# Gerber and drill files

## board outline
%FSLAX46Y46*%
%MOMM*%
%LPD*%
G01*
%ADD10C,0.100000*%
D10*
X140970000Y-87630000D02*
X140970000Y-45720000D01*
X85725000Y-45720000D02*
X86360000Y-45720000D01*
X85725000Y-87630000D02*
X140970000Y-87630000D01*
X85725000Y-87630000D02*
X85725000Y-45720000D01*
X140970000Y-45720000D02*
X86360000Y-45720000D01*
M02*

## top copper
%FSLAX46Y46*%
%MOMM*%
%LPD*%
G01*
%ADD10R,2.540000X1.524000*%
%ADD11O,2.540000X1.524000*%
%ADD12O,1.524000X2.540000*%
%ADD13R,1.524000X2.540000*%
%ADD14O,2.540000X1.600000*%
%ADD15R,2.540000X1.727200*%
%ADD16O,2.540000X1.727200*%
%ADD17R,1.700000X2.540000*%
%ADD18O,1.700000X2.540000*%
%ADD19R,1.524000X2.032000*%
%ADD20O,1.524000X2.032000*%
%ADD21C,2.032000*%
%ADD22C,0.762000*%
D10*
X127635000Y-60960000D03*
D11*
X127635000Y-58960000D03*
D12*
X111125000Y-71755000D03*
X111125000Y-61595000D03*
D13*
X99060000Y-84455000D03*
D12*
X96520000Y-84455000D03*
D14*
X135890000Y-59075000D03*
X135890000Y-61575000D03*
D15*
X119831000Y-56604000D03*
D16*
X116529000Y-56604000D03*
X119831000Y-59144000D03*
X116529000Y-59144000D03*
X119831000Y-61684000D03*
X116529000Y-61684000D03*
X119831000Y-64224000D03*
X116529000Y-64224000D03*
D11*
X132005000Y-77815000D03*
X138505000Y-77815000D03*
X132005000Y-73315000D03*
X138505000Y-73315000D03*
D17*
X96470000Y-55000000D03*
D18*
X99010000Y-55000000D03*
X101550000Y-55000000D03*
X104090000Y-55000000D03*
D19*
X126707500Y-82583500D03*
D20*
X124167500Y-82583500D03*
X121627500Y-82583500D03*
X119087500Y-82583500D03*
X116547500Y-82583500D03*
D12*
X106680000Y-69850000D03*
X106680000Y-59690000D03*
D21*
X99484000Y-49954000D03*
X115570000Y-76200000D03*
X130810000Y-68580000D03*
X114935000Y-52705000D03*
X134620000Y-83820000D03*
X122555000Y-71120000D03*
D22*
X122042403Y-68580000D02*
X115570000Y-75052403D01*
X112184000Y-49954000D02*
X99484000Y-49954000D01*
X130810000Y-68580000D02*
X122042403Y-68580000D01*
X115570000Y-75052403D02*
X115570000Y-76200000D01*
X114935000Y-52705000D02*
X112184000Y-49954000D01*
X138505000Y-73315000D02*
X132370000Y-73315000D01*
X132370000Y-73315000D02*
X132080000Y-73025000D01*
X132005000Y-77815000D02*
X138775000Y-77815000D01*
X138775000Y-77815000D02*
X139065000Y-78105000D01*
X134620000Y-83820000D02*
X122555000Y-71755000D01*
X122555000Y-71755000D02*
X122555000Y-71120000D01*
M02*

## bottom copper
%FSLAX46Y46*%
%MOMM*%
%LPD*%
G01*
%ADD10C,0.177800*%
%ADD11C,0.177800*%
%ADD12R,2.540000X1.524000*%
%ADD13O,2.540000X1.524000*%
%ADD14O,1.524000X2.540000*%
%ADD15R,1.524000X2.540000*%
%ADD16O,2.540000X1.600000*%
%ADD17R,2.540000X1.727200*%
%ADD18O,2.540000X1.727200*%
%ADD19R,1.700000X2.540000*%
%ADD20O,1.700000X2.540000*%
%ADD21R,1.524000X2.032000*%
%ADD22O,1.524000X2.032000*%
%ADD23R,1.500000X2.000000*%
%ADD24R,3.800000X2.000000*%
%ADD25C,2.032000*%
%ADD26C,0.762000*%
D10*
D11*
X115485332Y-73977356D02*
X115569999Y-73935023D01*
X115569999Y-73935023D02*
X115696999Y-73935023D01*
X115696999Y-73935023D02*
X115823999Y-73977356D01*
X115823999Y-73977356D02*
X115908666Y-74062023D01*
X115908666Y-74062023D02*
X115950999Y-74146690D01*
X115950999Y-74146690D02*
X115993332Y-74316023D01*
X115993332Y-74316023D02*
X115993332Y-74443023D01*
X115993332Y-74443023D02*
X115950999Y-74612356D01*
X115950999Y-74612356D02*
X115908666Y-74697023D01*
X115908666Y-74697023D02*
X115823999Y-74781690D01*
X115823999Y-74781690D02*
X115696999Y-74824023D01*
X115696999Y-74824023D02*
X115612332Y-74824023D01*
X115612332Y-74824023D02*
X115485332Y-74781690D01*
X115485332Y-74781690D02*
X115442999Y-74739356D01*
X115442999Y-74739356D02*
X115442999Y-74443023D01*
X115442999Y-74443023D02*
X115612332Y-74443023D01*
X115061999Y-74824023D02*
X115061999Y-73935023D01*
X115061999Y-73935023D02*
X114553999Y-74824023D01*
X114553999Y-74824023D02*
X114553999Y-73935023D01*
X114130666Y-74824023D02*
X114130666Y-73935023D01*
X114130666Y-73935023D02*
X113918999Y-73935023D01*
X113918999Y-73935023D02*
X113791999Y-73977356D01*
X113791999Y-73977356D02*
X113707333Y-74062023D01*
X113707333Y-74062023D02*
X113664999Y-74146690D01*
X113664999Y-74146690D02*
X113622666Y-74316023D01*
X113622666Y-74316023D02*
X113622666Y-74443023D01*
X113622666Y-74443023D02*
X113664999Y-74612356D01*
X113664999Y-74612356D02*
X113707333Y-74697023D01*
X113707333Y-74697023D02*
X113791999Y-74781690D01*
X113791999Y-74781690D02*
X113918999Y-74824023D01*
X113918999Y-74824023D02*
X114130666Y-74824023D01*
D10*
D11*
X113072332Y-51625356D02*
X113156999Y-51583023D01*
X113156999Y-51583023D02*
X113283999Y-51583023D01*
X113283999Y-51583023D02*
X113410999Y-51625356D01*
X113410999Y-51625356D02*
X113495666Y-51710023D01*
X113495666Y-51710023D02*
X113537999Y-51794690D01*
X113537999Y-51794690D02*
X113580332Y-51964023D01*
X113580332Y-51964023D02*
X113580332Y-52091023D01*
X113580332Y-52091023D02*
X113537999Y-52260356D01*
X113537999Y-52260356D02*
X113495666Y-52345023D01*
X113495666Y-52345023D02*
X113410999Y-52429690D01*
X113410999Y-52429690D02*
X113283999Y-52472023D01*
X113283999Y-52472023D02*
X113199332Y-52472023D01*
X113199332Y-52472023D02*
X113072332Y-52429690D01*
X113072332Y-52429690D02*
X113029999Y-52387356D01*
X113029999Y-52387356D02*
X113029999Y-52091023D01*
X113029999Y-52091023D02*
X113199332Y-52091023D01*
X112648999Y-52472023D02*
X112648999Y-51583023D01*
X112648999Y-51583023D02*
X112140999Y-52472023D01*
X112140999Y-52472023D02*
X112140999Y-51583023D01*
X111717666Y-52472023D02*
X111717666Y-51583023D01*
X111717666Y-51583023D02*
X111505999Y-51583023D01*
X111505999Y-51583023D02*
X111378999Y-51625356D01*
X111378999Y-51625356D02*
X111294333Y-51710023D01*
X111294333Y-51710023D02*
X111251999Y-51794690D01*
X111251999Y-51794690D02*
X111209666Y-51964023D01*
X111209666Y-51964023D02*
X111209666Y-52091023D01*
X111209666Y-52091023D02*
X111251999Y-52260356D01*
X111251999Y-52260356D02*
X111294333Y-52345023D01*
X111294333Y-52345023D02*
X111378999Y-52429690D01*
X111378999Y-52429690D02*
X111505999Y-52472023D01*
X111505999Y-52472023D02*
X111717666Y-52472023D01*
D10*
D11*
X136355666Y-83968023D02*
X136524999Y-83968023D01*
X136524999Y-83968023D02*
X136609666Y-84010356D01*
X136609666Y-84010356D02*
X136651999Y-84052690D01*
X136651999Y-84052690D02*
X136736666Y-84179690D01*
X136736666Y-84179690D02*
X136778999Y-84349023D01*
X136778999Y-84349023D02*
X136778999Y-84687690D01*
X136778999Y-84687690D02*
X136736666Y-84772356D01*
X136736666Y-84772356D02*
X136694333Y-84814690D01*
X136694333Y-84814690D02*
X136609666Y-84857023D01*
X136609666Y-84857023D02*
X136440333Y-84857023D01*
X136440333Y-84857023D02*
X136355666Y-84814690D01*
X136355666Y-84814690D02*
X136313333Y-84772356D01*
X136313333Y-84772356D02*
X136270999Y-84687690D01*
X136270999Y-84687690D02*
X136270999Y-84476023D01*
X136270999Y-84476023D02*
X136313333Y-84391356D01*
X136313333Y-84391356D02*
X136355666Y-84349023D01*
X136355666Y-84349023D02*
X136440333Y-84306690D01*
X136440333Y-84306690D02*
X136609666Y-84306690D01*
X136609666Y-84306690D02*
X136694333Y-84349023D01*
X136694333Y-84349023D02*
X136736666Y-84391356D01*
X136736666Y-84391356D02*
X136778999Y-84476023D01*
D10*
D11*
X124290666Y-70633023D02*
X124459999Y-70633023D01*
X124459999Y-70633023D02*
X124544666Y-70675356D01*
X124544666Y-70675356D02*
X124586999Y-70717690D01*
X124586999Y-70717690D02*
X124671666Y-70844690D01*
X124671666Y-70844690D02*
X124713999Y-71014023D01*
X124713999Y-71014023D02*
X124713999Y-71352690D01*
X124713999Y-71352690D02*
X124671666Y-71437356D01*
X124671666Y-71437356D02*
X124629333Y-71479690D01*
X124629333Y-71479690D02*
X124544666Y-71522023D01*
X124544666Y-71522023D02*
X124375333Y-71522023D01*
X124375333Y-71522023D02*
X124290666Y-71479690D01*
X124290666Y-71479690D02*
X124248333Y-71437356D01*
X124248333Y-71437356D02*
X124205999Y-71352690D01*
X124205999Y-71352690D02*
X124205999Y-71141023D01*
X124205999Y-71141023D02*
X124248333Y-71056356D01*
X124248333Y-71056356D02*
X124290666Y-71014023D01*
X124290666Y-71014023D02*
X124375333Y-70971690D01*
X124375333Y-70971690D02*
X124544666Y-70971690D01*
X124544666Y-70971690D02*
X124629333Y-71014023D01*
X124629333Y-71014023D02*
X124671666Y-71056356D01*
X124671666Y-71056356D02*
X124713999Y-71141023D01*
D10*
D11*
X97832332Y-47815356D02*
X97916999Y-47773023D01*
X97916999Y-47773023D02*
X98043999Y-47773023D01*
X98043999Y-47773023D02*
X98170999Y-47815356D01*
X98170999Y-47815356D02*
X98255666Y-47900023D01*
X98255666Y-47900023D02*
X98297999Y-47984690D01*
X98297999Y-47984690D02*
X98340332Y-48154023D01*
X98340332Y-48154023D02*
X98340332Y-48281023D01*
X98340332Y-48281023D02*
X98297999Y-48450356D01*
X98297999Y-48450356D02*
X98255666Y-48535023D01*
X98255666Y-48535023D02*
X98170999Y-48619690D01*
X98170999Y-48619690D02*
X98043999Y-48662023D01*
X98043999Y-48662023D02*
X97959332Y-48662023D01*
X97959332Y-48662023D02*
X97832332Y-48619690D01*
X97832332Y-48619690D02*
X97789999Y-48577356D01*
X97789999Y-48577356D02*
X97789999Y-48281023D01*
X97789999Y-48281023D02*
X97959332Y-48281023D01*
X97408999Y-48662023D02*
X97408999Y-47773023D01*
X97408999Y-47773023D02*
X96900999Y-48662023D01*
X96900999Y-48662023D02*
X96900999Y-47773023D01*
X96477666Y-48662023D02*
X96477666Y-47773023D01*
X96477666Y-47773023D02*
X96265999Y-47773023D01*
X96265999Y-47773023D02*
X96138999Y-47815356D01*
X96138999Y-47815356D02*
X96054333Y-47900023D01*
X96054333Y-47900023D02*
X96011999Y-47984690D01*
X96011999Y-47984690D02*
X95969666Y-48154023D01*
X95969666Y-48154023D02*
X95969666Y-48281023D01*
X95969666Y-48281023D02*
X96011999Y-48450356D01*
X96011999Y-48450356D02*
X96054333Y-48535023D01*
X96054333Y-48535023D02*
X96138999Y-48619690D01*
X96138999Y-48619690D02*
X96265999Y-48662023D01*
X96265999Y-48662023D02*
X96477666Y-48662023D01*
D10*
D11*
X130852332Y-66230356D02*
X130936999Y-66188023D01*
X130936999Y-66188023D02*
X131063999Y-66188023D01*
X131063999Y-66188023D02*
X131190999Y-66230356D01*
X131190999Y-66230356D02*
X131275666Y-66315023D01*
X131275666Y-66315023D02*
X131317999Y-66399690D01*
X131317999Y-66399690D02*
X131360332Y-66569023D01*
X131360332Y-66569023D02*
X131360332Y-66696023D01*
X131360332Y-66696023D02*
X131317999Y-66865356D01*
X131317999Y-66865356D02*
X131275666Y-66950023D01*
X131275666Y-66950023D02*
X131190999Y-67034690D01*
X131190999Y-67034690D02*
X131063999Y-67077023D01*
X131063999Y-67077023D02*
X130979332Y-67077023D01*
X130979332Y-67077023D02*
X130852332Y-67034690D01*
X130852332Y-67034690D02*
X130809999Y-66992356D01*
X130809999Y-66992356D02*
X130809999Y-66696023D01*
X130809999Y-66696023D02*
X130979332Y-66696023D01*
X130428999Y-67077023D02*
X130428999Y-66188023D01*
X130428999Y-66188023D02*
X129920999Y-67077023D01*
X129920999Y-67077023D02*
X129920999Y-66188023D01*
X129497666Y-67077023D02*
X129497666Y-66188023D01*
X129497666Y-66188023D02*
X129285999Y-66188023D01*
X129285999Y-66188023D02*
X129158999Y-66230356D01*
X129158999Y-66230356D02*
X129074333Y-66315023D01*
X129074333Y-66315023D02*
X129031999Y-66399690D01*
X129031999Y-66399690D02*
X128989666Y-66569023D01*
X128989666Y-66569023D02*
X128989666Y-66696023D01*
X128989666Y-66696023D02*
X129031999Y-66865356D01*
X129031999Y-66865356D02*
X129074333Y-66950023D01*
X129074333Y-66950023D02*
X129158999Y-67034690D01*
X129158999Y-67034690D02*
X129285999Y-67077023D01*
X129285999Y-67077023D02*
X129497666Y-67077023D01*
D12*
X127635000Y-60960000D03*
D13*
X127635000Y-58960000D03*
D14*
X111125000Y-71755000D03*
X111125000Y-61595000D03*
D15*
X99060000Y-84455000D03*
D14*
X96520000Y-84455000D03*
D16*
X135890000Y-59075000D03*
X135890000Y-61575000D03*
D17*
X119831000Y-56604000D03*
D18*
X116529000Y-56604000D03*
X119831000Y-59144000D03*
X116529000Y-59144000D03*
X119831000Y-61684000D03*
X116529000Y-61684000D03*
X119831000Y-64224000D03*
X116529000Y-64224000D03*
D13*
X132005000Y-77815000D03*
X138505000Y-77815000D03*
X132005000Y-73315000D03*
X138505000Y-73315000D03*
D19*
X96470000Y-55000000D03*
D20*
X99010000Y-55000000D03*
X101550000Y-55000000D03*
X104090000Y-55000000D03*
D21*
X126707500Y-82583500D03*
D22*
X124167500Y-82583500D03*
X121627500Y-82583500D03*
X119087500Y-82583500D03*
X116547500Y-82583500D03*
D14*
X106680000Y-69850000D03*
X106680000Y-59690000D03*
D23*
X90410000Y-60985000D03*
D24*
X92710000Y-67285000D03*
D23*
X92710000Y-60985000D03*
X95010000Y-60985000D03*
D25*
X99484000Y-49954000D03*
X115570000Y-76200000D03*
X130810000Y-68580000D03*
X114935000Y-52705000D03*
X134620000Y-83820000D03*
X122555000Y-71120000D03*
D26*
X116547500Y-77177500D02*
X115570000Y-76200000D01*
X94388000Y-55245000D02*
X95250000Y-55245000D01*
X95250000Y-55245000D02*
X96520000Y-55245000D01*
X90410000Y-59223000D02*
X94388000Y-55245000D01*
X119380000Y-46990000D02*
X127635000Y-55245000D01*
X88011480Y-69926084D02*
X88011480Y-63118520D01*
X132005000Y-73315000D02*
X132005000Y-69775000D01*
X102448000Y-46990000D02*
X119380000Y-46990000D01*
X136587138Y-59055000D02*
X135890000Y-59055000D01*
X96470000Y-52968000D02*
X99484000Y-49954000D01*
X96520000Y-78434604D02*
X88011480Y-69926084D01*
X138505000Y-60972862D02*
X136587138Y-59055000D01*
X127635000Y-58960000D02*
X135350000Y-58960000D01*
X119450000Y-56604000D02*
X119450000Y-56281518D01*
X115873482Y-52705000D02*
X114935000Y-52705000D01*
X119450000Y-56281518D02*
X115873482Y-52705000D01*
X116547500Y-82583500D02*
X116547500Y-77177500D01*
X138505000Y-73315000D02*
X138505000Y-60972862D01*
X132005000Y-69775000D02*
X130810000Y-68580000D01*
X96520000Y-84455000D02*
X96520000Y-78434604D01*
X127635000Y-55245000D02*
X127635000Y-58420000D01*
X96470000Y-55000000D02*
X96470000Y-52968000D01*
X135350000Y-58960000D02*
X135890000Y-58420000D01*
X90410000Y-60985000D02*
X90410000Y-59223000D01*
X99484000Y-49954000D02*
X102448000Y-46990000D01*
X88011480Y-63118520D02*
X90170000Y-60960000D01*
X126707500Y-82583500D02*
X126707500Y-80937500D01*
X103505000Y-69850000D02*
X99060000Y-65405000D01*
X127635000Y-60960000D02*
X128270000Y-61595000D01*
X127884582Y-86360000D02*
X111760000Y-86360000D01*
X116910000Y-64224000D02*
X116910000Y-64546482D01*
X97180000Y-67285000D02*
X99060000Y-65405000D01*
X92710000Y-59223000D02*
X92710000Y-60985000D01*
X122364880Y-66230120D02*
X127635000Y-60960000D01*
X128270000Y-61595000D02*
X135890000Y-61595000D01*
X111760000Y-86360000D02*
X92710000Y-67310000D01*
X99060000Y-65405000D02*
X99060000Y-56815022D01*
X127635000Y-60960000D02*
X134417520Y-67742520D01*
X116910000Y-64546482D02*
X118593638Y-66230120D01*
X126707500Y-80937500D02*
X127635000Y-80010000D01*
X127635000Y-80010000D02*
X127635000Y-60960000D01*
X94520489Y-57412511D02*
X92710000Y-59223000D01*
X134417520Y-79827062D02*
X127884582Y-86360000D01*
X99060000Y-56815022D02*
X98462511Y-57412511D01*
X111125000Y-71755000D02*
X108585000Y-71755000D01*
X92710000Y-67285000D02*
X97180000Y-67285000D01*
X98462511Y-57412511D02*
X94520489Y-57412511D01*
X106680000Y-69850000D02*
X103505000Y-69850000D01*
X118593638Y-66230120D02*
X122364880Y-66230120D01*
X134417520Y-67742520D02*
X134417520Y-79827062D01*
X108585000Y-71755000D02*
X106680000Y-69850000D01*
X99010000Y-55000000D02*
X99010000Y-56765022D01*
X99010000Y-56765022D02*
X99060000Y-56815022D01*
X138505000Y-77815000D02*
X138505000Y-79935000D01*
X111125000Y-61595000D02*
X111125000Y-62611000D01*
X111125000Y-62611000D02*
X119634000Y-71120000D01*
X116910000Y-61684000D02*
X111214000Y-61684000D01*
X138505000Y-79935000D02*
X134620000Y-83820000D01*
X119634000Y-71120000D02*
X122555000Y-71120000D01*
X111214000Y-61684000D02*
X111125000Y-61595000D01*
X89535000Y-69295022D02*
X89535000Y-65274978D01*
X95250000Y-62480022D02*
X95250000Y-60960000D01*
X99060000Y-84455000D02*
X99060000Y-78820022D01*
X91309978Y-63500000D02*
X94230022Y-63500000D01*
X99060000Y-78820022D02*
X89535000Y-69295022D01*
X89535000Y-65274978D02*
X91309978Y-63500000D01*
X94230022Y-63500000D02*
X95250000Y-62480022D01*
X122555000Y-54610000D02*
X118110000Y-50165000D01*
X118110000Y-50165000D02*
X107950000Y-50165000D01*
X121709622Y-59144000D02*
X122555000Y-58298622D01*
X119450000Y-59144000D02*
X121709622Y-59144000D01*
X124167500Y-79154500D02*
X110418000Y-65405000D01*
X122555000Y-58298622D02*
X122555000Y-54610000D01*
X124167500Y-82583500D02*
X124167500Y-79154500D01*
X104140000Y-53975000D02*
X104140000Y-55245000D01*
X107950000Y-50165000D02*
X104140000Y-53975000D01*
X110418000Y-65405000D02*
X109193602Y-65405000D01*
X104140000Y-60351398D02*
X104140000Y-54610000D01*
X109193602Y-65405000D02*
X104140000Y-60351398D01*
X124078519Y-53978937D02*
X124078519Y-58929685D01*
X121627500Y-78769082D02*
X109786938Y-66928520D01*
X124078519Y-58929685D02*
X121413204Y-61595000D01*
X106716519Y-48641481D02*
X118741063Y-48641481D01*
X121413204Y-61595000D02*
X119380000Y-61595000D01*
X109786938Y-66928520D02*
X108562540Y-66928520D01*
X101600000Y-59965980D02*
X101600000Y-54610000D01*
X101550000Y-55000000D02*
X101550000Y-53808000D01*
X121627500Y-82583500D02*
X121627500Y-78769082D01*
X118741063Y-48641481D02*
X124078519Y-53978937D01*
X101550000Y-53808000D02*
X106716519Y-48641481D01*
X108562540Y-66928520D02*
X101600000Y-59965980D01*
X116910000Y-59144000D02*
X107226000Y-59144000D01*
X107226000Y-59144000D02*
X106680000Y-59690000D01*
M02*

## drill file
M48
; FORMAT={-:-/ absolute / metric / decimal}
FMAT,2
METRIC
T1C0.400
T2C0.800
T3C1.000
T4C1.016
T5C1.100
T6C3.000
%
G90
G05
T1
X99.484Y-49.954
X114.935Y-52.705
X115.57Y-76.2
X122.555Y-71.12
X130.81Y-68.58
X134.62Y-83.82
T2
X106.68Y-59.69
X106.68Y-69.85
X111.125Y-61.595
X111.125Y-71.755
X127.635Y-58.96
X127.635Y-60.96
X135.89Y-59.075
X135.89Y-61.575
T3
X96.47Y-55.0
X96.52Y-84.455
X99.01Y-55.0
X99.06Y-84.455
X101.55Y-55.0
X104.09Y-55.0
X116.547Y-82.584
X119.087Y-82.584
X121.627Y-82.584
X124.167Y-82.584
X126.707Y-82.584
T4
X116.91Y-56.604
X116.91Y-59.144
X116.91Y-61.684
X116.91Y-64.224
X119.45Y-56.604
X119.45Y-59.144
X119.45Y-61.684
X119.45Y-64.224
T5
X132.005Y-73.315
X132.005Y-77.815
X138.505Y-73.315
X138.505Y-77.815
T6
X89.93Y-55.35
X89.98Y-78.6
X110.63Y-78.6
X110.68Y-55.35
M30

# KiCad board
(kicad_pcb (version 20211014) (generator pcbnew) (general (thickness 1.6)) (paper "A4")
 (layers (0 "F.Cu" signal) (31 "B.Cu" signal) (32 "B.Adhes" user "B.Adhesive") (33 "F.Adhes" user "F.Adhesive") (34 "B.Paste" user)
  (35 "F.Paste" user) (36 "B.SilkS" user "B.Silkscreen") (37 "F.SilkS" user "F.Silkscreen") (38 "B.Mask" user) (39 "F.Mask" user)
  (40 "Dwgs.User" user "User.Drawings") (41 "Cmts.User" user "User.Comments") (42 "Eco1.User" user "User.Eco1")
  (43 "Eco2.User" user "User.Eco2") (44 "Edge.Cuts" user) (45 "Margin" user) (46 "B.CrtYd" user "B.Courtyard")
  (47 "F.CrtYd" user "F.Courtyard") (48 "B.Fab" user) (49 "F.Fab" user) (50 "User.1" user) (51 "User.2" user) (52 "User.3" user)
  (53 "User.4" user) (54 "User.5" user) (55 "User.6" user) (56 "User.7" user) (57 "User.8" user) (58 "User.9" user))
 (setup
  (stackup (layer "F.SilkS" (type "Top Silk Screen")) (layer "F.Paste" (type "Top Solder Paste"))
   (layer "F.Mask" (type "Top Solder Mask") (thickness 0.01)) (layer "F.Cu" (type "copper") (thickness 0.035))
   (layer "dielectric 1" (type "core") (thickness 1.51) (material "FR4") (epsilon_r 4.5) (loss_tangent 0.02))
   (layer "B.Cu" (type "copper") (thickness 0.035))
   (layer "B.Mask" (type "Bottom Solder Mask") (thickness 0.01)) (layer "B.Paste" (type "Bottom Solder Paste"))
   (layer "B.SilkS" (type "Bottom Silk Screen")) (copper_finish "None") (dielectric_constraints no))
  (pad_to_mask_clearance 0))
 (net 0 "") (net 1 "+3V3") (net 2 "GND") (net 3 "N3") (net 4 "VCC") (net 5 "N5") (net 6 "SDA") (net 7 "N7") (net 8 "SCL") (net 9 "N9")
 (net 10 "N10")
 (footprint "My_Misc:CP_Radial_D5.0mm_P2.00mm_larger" (layer "F.Cu") (at 127.635 60.96 90)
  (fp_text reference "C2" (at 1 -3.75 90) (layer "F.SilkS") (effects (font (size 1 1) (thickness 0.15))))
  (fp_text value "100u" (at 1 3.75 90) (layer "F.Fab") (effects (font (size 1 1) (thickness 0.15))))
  (pad "1" thru_hole rect (at 0 0 90) (size 1.524 2.54) (drill 0.8) (layers *.Cu *.Mask) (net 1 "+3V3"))
  (pad "2" thru_hole oval (at 2 0 90) (size 1.524 2.54) (drill 0.8) (layers *.Cu *.Mask) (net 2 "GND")))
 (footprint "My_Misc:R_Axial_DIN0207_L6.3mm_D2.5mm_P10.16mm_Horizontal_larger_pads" (layer "F.Cu") (at 111.125 71.755 90)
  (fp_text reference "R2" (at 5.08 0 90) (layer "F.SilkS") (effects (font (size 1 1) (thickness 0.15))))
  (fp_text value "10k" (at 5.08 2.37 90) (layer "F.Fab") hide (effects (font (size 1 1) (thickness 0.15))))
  (pad "1" thru_hole oval (at 0 0 90) (size 2.54 1.524) (drill 0.8) (layers *.Cu *.Mask) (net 1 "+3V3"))
  (pad "2" thru_hole oval (at 10.16 0 90) (size 2.54 1.524) (drill 0.8) (layers *.Cu *.Mask) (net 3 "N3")))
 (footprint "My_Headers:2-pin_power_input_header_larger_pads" (layer "F.Cu") (at 99.06 84.455 -90)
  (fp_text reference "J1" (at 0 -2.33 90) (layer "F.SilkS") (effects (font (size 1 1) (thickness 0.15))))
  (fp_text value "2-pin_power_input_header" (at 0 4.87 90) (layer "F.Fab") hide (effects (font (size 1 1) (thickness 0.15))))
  (pad "1" thru_hole rect locked (at 0 0 270) (size 2.54 1.524) (drill 1) (layers *.Cu *.Mask) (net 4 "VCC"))
  (pad "2" thru_hole oval locked (at 0 2.54 270) (size 2.54 1.524) (drill 1) (layers *.Cu *.Mask) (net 2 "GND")))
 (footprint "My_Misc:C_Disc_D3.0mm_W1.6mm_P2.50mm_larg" (layer "F.Cu") (at 135.89 59.075 -90)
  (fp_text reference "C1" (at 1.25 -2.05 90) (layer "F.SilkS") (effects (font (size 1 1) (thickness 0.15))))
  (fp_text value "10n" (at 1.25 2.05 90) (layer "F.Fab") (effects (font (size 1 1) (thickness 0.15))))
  (pad "1" thru_hole oval locked (at 0 0 270) (size 1.6 2.54) (drill 0.8) (layers *.Cu *.Mask) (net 2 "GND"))
  (pad "2" thru_hole oval locked (at 2.5 0 270) (size 1.6 2.54) (drill 0.8) (layers *.Cu *.Mask) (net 1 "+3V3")))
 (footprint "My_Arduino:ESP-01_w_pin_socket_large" (layer "F.Cu") (at 116.91 56.604)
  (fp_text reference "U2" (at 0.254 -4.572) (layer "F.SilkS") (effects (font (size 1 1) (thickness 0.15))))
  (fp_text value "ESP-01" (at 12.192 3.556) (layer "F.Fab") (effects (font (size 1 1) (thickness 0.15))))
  (pad "1" thru_hole rect (at 2.54 0) (size 2.54 1.7272) (drill 1.016 (offset 0.381 0)) (layers *.Cu *.Mask) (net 2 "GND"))
  (pad "2" thru_hole oval (at 0 0) (size 2.54 1.7272) (drill 1.016 (offset -0.381 0)) (layers *.Cu *.Mask) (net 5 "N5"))
  (pad "3" thru_hole oval (at 2.54 2.54) (size 2.54 1.7272) (drill 1.016 (offset 0.381 0)) (layers *.Cu *.Mask) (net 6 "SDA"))
  (pad "4" thru_hole oval (at 0 2.54) (size 2.54 1.7272) (drill 1.016 (offset -0.381 0)) (layers *.Cu *.Mask) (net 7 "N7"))
  (pad "5" thru_hole oval (at 2.54 5.08) (size 2.54 1.7272) (drill 1.016 (offset 0.381 0)) (layers *.Cu *.Mask) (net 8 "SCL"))
  (pad "6" thru_hole oval (at 0 5.08) (size 2.54 1.7272) (drill 1.016 (offset -0.381 0)) (layers *.Cu *.Mask) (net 3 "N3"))
  (pad "7" thru_hole oval (at 2.54 7.62) (size 2.54 1.7272) (drill 1.016 (offset 0.381 0)) (layers *.Cu *.Mask) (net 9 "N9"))
  (pad "8" thru_hole oval (at 0 7.62) (size 2.54 1.7272) (drill 1.016 (offset -0.381 0)) (layers *.Cu *.Mask) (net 1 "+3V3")))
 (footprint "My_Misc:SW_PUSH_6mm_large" (layer "F.Cu") (at 138.505 77.815 180)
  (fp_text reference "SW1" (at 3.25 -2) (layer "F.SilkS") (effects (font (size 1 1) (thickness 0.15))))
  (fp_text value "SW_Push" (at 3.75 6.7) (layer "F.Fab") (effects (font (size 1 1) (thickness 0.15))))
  (pad "1" thru_hole oval locked (at 6.5 0 270) (size 1.524 2.54) (drill 1.1) (layers *.Cu *.Mask) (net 3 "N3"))
  (pad "1" thru_hole oval locked (at 0 0 270) (size 1.524 2.54) (drill 1.1) (layers *.Cu *.Mask) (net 3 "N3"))
  (pad "2" thru_hole oval locked (at 6.5 4.5 270) (size 1.524 2.54) (drill 1.1) (layers *.Cu *.Mask) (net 2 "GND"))
  (pad "2" thru_hole oval locked (at 0 4.5 270) (size 1.524 2.54) (drill 1.1) (layers *.Cu *.Mask) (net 2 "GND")))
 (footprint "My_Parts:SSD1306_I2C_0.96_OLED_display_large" (layer "F.Cu") (at 96.47 55)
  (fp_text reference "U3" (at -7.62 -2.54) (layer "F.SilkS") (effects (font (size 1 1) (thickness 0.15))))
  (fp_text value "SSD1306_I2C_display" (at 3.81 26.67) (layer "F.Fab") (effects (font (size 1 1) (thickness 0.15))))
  (pad "" np_thru_hole oval (at -6.49 23.6) (size 3 3) (drill 3) (layers *.Cu *.Mask))
  (pad "" np_thru_hole oval (at 14.16 23.6) (size 3 3) (drill 3) (layers *.Cu *.Mask))
  (pad "" np_thru_hole oval (at 14.21 0.35) (size 3 3) (drill 3) (layers *.Cu *.Mask))
  (pad "" np_thru_hole oval (at -6.54 0.35) (size 3 3) (drill 3) (layers *.Cu *.Mask))
  (pad "1" thru_hole rect (at 0 0 90) (size 2.54 1.7) (drill 1) (layers *.Cu *.Mask) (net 2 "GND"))
  (pad "2" thru_hole oval (at 2.54 0 90) (size 2.54 1.7) (drill 1) (layers *.Cu *.Mask) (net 1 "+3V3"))
  (pad "3" thru_hole oval (at 5.08 0 90) (size 2.54 1.7) (drill 1) (layers *.Cu *.Mask) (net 8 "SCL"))
  (pad "4" thru_hole oval (at 7.62 0 90) (size 2.54 1.7) (drill 1) (layers *.Cu *.Mask) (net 6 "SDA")))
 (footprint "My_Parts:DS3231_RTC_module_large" (layer "F.Cu") (at 116.5475 82.5835 90)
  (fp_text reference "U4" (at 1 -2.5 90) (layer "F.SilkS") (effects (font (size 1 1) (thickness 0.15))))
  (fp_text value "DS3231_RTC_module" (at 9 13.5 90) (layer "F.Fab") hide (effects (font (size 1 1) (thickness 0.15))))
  (pad "1" thru_hole rect (at 0 10.16 270) (size 2.032 1.524) (drill 1) (layers *.Cu *.Mask) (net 1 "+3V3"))
  (pad "2" thru_hole oval (at 0 7.62 270) (size 2.032 1.524) (drill 1) (layers *.Cu *.Mask) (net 6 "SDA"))
  (pad "3" thru_hole oval (at 0 5.08 270) (size 2.032 1.524) (drill 1) (layers *.Cu *.Mask) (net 8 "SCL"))
  (pad "4" thru_hole oval (at 0 2.54 270) (size 2.032 1.524) (drill 1) (layers *.Cu *.Mask) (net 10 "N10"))
  (pad "5" thru_hole oval (at 0 0 270) (size 2.032 1.524) (drill 1) (layers *.Cu *.Mask) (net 2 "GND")))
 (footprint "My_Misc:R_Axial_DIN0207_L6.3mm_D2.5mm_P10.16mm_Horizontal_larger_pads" (layer "F.Cu") (at 106.68 69.85 90)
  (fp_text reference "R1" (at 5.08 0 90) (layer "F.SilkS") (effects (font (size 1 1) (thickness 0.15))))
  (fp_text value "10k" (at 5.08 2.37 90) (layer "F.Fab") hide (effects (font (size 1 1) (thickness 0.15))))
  (pad "1" thru_hole oval (at 0 0 90) (size 2.54 1.524) (drill 0.8) (layers *.Cu *.Mask) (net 1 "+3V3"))
  (pad "2" thru_hole oval (at 10.16 0 90) (size 2.54 1.524) (drill 0.8) (layers *.Cu *.Mask) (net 7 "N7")))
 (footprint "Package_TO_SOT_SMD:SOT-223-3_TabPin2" (layer "B.Cu") (at 92.71 64.135 -90)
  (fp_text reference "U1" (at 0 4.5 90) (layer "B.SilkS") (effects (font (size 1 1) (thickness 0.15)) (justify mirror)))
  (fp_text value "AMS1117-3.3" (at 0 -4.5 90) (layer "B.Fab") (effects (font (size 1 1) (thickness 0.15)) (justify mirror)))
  (pad "1" smd rect (at -3.15 2.3 270) (size 2 1.5) (layers "B.Cu" "B.Paste" "B.Mask") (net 2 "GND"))
  (pad "2" smd rect (at 3.15 0 270) (size 2 3.8) (layers "B.Cu" "B.Paste" "B.Mask") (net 1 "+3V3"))
  (pad "2" smd rect (at -3.15 0 270) (size 2 1.5) (layers "B.Cu" "B.Paste" "B.Mask") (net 1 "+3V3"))
  (pad "3" smd rect (at -3.15 -2.3 270) (size 2 1.5) (layers "B.Cu" "B.Paste" "B.Mask") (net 4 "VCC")))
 (gr_line (start 140.97 87.63) (end 140.97 45.72) (layer "Edge.Cuts") (width 0.1))
 (gr_line (start 85.725 45.72) (end 86.36 45.72) (layer "Edge.Cuts") (width 0.1))
 (gr_line (start 85.725 87.63) (end 140.97 87.63) (layer "Edge.Cuts") (width 0.1))
 (gr_line (start 85.725 87.63) (end 85.725 45.72) (layer "Edge.Cuts") (width 0.1))
 (gr_line (start 140.97 45.72) (end 86.36 45.72) (layer "Edge.Cuts") (width 0.1))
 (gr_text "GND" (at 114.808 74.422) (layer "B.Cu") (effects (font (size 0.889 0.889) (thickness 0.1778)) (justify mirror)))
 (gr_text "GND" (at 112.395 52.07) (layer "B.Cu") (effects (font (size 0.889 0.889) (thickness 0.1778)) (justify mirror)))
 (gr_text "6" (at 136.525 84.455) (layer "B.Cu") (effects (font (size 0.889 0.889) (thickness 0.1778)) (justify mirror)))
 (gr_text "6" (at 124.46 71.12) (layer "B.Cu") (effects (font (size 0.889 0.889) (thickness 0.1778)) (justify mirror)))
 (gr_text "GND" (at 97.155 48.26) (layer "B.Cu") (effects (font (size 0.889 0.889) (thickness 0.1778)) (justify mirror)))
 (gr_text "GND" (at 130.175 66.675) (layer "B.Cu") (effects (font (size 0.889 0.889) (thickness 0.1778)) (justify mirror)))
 (segment (start 122.042403 68.58) (end 115.57 75.052403) (width 0.762) (layer "F.Cu") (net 2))
 (segment (start 112.184 49.954) (end 99.484 49.954) (width 0.762) (layer "F.Cu") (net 2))
 (segment (start 130.81 68.58) (end 122.042403 68.58) (width 0.762) (layer "F.Cu") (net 2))
 (segment (start 115.57 75.052403) (end 115.57 76.2) (width 0.762) (layer "F.Cu") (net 2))
 (segment (start 114.935 52.705) (end 112.184 49.954) (width 0.762) (layer "F.Cu") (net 2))
 (segment (start 138.505 73.315) (end 132.37 73.315) (width 0.762) (layer "F.Cu") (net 2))
 (segment (start 132.37 73.315) (end 132.08 73.025) (width 0.762) (layer "F.Cu") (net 2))
 (via (at 99.484 49.954) (size 2.032) (drill 0.4) (layers "F.Cu" "B.Cu") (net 2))
 (via (at 115.57 76.2) (size 2.032) (drill 0.4) (layers "F.Cu" "B.Cu") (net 2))
 (via (at 130.81 68.58) (size 2.032) (drill 0.4) (layers "F.Cu" "B.Cu") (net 2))
 (via (at 114.935 52.705) (size 2.032) (drill 0.4) (layers "F.Cu" "B.Cu") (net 2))
 (segment (start 116.5475 77.1775) (end 115.57 76.2) (width 0.762) (layer "B.Cu") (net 2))
 (segment (start 94.388 55.245) (end 95.25 55.245) (width 0.762) (layer "B.Cu") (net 2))
 (segment (start 95.25 55.245) (end 96.52 55.245) (width 0.762) (layer "B.Cu") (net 2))
 (segment (start 90.41 59.223) (end 94.388 55.245) (width 0.762) (layer "B.Cu") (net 2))
 (segment (start 119.38 46.99) (end 127.635 55.245) (width 0.762) (layer "B.Cu") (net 2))
 (segment (start 88.01148 69.926084) (end 88.01148 63.11852) (width 0.762) (layer "B.Cu") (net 2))
 (segment (start 132.005 73.315) (end 132.005 69.775) (width 0.762) (layer "B.Cu") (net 2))
 (segment (start 102.448 46.99) (end 119.38 46.99) (width 0.762) (layer "B.Cu") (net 2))
 (segment (start 136.587138 59.055) (end 135.89 59.055) (width 0.762) (layer "B.Cu") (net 2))
 (segment (start 96.47 52.968) (end 99.484 49.954) (width 0.762) (layer "B.Cu") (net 2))
 (segment (start 96.52 78.434604) (end 88.01148 69.926084) (width 0.762) (layer "B.Cu") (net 2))
 (segment (start 138.505 60.972862) (end 136.587138 59.055) (width 0.762) (layer "B.Cu") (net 2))
 (segment (start 127.635 58.96) (end 135.35 58.96) (width 0.762) (layer "B.Cu") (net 2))
 (segment (start 119.45 56.604) (end 119.45 56.281518) (width 0.762) (layer "B.Cu") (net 2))
 (segment (start 115.873482 52.705) (end 114.935 52.705) (width 0.762) (layer "B.Cu") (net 2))
 (segment (start 119.45 56.281518) (end 115.873482 52.705) (width 0.762) (layer "B.Cu") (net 2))
 (segment (start 116.5475 82.5835) (end 116.5475 77.1775) (width 0.762) (layer "B.Cu") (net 2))
 (segment (start 138.505 73.315) (end 138.505 60.972862) (width 0.762) (layer "B.Cu") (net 2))
 (segment (start 132.005 69.775) (end 130.81 68.58) (width 0.762) (layer "B.Cu") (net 2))
 (segment (start 96.52 84.455) (end 96.52 78.434604) (width 0.762) (layer "B.Cu") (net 2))
 (segment (start 127.635 55.245) (end 127.635 58.42) (width 0.762) (layer "B.Cu") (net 2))
 (segment (start 96.47 55) (end 96.47 52.968) (width 0.762) (layer "B.Cu") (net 2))
 (segment (start 135.35 58.96) (end 135.89 58.42) (width 0.762) (layer "B.Cu") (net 2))
 (segment (start 90.41 60.985) (end 90.41 59.223) (width 0.762) (layer "B.Cu") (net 2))
 (segment (start 99.484 49.954) (end 102.448 46.99) (width 0.762) (layer "B.Cu") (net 2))
 (segment (start 88.01148 63.11852) (end 90.17 60.96) (width 0.762) (layer "B.Cu") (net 2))
 (segment (start 126.7075 82.5835) (end 126.7075 80.9375) (width 0.762) (layer "B.Cu") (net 1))
 (segment (start 103.505 69.85) (end 99.06 65.405) (width 0.762) (layer "B.Cu") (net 1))
 (segment (start 127.635 60.96) (end 128.27 61.595) (width 0.762) (layer "B.Cu") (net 1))
 (segment (start 127.884582 86.36) (end 111.76 86.36) (width 0.762) (layer "B.Cu") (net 1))
 (segment (start 116.91 64.224) (end 116.91 64.546482) (width 0.762) (layer "B.Cu") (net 1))
 (segment (start 97.18 67.285) (end 99.06 65.405) (width 0.762) (layer "B.Cu") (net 1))
 (segment (start 92.71 59.223) (end 92.71 60.985) (width 0.762) (layer "B.Cu") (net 1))
 (segment (start 122.36488 66.23012) (end 127.635 60.96) (width 0.762) (layer "B.Cu") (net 1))
 (segment (start 128.27 61.595) (end 135.89 61.595) (width 0.762) (layer "B.Cu") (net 1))
 (segment (start 111.76 86.36) (end 92.71 67.31) (width 0.762) (layer "B.Cu") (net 1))
 (segment (start 99.06 65.405) (end 99.06 56.815022) (width 0.762) (layer "B.Cu") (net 1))
 (segment (start 127.635 60.96) (end 134.41752 67.74252) (width 0.762) (layer "B.Cu") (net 1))
 (segment (start 116.91 64.546482) (end 118.593638 66.23012) (width 0.762) (layer "B.Cu") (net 1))
 (segment (start 126.7075 80.9375) (end 127.635 80.01) (width 0.762) (layer "B.Cu") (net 1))
 (segment (start 127.635 80.01) (end 127.635 60.96) (width 0.762) (layer "B.Cu") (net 1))
 (segment (start 94.520489 57.412511) (end 92.71 59.223) (width 0.762) (layer "B.Cu") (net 1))
 (segment (start 134.41752 79.827062) (end 127.884582 86.36) (width 0.762) (layer "B.Cu") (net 1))
 (segment (start 99.06 56.815022) (end 98.462511 57.412511) (width 0.762) (layer "B.Cu") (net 1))
 (segment (start 111.125 71.755) (end 108.585 71.755) (width 0.762) (layer "B.Cu") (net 1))
 (segment (start 92.71 67.285) (end 97.18 67.285) (width 0.762) (layer "B.Cu") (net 1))
 (segment (start 98.462511 57.412511) (end 94.520489 57.412511) (width 0.762) (layer "B.Cu") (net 1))
 (segment (start 106.68 69.85) (end 103.505 69.85) (width 0.762) (layer "B.Cu") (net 1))
 (segment (start 118.593638 66.23012) (end 122.36488 66.23012) (width 0.762) (layer "B.Cu") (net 1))
 (segment (start 134.41752 67.74252) (end 134.41752 79.827062) (width 0.762) (layer "B.Cu") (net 1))
 (segment (start 108.585 71.755) (end 106.68 69.85) (width 0.762) (layer "B.Cu") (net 1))
 (segment (start 99.01 55) (end 99.01 56.765022) (width 0.762) (layer "B.Cu") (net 1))
 (segment (start 99.01 56.765022) (end 99.06 56.815022) (width 0.762) (layer "B.Cu") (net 1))
 (segment (start 132.005 77.815) (end 138.775 77.815) (width 0.762) (layer "F.Cu") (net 3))
 (segment (start 138.775 77.815) (end 139.065 78.105) (width 0.762) (layer "F.Cu") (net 3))
 (segment (start 134.62 83.82) (end 122.555 71.755) (width 0.762) (layer "F.Cu") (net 3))
 (segment (start 122.555 71.755) (end 122.555 71.12) (width 0.762) (layer "F.Cu") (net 3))
 (via (at 134.62 83.82) (size 2.032) (drill 0.4) (layers "F.Cu" "B.Cu") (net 3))
 (via (at 122.555 71.12) (size 2.032) (drill 0.4) (layers "F.Cu" "B.Cu") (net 3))
 (segment (start 138.505 77.815) (end 138.505 79.935) (width 0.762) (layer "B.Cu") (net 3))
 (segment (start 111.125 61.595) (end 111.125 62.611) (width 0.762) (layer "B.Cu") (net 3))
 (segment (start 111.125 62.611) (end 119.634 71.12) (width 0.762) (layer "B.Cu") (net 3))
 (segment (start 116.91 61.684) (end 111.214 61.684) (width 0.762) (layer "B.Cu") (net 3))
 (segment (start 138.505 79.935) (end 134.62 83.82) (width 0.762) (layer "B.Cu") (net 3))
 (segment (start 119.634 71.12) (end 122.555 71.12) (width 0.762) (layer "B.Cu") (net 3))
 (segment (start 111.214 61.684) (end 111.125 61.595) (width 0.762) (layer "B.Cu") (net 3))
 (segment (start 89.535 69.295022) (end 89.535 65.274978) (width 0.762) (layer "B.Cu") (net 4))
 (segment (start 95.25 62.480022) (end 95.25 60.96) (width 0.762) (layer "B.Cu") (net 4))
 (segment (start 99.06 84.455) (end 99.06 78.820022) (width 0.762) (layer "B.Cu") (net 4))
 (segment (start 91.309978 63.5) (end 94.230022 63.5) (width 0.762) (layer "B.Cu") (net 4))
 (segment (start 99.06 78.820022) (end 89.535 69.295022) (width 0.762) (layer "B.Cu") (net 4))
 (segment (start 89.535 65.274978) (end 91.309978 63.5) (width 0.762) (layer "B.Cu") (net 4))
 (segment (start 94.230022 63.5) (end 95.25 62.480022) (width 0.762) (layer "B.Cu") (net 4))
 (segment (start 122.555 54.61) (end 118.11 50.165) (width 0.762) (layer "B.Cu") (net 6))
 (segment (start 118.11 50.165) (end 107.95 50.165) (width 0.762) (layer "B.Cu") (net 6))
 (segment (start 121.709622 59.144) (end 122.555 58.298622) (width 0.762) (layer "B.Cu") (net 6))
 (segment (start 119.45 59.144) (end 121.709622 59.144) (width 0.762) (layer "B.Cu") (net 6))
 (segment (start 124.1675 79.1545) (end 110.418 65.405) (width 0.762) (layer "B.Cu") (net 6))
 (segment (start 122.555 58.298622) (end 122.555 54.61) (width 0.762) (layer "B.Cu") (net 6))
 (segment (start 124.1675 82.5835) (end 124.1675 79.1545) (width 0.762) (layer "B.Cu") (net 6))
 (segment (start 104.14 53.975) (end 104.14 55.245) (width 0.762) (layer "B.Cu") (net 6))
 (segment (start 107.95 50.165) (end 104.14 53.975) (width 0.762) (layer "B.Cu") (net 6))
 (segment (start 110.418 65.405) (end 109.193602 65.405) (width 0.762) (layer "B.Cu") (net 6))
 (segment (start 104.14 60.351398) (end 104.14 54.61) (width 0.762) (layer "B.Cu") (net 6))
 (segment (start 109.193602 65.405) (end 104.14 60.351398) (width 0.762) (layer "B.Cu") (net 6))
 (segment (start 124.078519 53.978937) (end 124.078519 58.929685) (width 0.762) (layer "B.Cu") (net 8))
 (segment (start 121.6275 78.769082) (end 109.786938 66.92852) (width 0.762) (layer "B.Cu") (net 8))
 (segment (start 124.078519 58.929685) (end 121.413204 61.595) (width 0.762) (layer "B.Cu") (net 8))
 (segment (start 106.716519 48.641481) (end 118.741063 48.641481) (width 0.762) (layer "B.Cu") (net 8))
 (segment (start 121.413204 61.595) (end 119.38 61.595) (width 0.762) (layer "B.Cu") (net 8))
 (segment (start 109.786938 66.92852) (end 108.56254 66.92852) (width 0.762) (layer "B.Cu") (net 8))
 (segment (start 101.6 59.96598) (end 101.6 54.61) (width 0.762) (layer "B.Cu") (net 8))
 (segment (start 101.55 55) (end 101.55 53.808) (width 0.762) (layer "B.Cu") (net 8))
 (segment (start 121.6275 82.5835) (end 121.6275 78.769082) (width 0.762) (layer "B.Cu") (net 8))
 (segment (start 118.741063 48.641481) (end 124.078519 53.978937) (width 0.762) (layer "B.Cu") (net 8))
 (segment (start 101.55 53.808) (end 106.716519 48.641481) (width 0.762) (layer "B.Cu") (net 8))
 (segment (start 108.56254 66.92852) (end 101.6 59.96598) (width 0.762) (layer "B.Cu") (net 8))
 (segment (start 116.91 59.144) (end 107.226 59.144) (width 0.762) (layer "B.Cu") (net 7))
 (segment (start 107.226 59.144) (end 106.68 59.69) (width 0.762) (layer "B.Cu") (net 7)))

